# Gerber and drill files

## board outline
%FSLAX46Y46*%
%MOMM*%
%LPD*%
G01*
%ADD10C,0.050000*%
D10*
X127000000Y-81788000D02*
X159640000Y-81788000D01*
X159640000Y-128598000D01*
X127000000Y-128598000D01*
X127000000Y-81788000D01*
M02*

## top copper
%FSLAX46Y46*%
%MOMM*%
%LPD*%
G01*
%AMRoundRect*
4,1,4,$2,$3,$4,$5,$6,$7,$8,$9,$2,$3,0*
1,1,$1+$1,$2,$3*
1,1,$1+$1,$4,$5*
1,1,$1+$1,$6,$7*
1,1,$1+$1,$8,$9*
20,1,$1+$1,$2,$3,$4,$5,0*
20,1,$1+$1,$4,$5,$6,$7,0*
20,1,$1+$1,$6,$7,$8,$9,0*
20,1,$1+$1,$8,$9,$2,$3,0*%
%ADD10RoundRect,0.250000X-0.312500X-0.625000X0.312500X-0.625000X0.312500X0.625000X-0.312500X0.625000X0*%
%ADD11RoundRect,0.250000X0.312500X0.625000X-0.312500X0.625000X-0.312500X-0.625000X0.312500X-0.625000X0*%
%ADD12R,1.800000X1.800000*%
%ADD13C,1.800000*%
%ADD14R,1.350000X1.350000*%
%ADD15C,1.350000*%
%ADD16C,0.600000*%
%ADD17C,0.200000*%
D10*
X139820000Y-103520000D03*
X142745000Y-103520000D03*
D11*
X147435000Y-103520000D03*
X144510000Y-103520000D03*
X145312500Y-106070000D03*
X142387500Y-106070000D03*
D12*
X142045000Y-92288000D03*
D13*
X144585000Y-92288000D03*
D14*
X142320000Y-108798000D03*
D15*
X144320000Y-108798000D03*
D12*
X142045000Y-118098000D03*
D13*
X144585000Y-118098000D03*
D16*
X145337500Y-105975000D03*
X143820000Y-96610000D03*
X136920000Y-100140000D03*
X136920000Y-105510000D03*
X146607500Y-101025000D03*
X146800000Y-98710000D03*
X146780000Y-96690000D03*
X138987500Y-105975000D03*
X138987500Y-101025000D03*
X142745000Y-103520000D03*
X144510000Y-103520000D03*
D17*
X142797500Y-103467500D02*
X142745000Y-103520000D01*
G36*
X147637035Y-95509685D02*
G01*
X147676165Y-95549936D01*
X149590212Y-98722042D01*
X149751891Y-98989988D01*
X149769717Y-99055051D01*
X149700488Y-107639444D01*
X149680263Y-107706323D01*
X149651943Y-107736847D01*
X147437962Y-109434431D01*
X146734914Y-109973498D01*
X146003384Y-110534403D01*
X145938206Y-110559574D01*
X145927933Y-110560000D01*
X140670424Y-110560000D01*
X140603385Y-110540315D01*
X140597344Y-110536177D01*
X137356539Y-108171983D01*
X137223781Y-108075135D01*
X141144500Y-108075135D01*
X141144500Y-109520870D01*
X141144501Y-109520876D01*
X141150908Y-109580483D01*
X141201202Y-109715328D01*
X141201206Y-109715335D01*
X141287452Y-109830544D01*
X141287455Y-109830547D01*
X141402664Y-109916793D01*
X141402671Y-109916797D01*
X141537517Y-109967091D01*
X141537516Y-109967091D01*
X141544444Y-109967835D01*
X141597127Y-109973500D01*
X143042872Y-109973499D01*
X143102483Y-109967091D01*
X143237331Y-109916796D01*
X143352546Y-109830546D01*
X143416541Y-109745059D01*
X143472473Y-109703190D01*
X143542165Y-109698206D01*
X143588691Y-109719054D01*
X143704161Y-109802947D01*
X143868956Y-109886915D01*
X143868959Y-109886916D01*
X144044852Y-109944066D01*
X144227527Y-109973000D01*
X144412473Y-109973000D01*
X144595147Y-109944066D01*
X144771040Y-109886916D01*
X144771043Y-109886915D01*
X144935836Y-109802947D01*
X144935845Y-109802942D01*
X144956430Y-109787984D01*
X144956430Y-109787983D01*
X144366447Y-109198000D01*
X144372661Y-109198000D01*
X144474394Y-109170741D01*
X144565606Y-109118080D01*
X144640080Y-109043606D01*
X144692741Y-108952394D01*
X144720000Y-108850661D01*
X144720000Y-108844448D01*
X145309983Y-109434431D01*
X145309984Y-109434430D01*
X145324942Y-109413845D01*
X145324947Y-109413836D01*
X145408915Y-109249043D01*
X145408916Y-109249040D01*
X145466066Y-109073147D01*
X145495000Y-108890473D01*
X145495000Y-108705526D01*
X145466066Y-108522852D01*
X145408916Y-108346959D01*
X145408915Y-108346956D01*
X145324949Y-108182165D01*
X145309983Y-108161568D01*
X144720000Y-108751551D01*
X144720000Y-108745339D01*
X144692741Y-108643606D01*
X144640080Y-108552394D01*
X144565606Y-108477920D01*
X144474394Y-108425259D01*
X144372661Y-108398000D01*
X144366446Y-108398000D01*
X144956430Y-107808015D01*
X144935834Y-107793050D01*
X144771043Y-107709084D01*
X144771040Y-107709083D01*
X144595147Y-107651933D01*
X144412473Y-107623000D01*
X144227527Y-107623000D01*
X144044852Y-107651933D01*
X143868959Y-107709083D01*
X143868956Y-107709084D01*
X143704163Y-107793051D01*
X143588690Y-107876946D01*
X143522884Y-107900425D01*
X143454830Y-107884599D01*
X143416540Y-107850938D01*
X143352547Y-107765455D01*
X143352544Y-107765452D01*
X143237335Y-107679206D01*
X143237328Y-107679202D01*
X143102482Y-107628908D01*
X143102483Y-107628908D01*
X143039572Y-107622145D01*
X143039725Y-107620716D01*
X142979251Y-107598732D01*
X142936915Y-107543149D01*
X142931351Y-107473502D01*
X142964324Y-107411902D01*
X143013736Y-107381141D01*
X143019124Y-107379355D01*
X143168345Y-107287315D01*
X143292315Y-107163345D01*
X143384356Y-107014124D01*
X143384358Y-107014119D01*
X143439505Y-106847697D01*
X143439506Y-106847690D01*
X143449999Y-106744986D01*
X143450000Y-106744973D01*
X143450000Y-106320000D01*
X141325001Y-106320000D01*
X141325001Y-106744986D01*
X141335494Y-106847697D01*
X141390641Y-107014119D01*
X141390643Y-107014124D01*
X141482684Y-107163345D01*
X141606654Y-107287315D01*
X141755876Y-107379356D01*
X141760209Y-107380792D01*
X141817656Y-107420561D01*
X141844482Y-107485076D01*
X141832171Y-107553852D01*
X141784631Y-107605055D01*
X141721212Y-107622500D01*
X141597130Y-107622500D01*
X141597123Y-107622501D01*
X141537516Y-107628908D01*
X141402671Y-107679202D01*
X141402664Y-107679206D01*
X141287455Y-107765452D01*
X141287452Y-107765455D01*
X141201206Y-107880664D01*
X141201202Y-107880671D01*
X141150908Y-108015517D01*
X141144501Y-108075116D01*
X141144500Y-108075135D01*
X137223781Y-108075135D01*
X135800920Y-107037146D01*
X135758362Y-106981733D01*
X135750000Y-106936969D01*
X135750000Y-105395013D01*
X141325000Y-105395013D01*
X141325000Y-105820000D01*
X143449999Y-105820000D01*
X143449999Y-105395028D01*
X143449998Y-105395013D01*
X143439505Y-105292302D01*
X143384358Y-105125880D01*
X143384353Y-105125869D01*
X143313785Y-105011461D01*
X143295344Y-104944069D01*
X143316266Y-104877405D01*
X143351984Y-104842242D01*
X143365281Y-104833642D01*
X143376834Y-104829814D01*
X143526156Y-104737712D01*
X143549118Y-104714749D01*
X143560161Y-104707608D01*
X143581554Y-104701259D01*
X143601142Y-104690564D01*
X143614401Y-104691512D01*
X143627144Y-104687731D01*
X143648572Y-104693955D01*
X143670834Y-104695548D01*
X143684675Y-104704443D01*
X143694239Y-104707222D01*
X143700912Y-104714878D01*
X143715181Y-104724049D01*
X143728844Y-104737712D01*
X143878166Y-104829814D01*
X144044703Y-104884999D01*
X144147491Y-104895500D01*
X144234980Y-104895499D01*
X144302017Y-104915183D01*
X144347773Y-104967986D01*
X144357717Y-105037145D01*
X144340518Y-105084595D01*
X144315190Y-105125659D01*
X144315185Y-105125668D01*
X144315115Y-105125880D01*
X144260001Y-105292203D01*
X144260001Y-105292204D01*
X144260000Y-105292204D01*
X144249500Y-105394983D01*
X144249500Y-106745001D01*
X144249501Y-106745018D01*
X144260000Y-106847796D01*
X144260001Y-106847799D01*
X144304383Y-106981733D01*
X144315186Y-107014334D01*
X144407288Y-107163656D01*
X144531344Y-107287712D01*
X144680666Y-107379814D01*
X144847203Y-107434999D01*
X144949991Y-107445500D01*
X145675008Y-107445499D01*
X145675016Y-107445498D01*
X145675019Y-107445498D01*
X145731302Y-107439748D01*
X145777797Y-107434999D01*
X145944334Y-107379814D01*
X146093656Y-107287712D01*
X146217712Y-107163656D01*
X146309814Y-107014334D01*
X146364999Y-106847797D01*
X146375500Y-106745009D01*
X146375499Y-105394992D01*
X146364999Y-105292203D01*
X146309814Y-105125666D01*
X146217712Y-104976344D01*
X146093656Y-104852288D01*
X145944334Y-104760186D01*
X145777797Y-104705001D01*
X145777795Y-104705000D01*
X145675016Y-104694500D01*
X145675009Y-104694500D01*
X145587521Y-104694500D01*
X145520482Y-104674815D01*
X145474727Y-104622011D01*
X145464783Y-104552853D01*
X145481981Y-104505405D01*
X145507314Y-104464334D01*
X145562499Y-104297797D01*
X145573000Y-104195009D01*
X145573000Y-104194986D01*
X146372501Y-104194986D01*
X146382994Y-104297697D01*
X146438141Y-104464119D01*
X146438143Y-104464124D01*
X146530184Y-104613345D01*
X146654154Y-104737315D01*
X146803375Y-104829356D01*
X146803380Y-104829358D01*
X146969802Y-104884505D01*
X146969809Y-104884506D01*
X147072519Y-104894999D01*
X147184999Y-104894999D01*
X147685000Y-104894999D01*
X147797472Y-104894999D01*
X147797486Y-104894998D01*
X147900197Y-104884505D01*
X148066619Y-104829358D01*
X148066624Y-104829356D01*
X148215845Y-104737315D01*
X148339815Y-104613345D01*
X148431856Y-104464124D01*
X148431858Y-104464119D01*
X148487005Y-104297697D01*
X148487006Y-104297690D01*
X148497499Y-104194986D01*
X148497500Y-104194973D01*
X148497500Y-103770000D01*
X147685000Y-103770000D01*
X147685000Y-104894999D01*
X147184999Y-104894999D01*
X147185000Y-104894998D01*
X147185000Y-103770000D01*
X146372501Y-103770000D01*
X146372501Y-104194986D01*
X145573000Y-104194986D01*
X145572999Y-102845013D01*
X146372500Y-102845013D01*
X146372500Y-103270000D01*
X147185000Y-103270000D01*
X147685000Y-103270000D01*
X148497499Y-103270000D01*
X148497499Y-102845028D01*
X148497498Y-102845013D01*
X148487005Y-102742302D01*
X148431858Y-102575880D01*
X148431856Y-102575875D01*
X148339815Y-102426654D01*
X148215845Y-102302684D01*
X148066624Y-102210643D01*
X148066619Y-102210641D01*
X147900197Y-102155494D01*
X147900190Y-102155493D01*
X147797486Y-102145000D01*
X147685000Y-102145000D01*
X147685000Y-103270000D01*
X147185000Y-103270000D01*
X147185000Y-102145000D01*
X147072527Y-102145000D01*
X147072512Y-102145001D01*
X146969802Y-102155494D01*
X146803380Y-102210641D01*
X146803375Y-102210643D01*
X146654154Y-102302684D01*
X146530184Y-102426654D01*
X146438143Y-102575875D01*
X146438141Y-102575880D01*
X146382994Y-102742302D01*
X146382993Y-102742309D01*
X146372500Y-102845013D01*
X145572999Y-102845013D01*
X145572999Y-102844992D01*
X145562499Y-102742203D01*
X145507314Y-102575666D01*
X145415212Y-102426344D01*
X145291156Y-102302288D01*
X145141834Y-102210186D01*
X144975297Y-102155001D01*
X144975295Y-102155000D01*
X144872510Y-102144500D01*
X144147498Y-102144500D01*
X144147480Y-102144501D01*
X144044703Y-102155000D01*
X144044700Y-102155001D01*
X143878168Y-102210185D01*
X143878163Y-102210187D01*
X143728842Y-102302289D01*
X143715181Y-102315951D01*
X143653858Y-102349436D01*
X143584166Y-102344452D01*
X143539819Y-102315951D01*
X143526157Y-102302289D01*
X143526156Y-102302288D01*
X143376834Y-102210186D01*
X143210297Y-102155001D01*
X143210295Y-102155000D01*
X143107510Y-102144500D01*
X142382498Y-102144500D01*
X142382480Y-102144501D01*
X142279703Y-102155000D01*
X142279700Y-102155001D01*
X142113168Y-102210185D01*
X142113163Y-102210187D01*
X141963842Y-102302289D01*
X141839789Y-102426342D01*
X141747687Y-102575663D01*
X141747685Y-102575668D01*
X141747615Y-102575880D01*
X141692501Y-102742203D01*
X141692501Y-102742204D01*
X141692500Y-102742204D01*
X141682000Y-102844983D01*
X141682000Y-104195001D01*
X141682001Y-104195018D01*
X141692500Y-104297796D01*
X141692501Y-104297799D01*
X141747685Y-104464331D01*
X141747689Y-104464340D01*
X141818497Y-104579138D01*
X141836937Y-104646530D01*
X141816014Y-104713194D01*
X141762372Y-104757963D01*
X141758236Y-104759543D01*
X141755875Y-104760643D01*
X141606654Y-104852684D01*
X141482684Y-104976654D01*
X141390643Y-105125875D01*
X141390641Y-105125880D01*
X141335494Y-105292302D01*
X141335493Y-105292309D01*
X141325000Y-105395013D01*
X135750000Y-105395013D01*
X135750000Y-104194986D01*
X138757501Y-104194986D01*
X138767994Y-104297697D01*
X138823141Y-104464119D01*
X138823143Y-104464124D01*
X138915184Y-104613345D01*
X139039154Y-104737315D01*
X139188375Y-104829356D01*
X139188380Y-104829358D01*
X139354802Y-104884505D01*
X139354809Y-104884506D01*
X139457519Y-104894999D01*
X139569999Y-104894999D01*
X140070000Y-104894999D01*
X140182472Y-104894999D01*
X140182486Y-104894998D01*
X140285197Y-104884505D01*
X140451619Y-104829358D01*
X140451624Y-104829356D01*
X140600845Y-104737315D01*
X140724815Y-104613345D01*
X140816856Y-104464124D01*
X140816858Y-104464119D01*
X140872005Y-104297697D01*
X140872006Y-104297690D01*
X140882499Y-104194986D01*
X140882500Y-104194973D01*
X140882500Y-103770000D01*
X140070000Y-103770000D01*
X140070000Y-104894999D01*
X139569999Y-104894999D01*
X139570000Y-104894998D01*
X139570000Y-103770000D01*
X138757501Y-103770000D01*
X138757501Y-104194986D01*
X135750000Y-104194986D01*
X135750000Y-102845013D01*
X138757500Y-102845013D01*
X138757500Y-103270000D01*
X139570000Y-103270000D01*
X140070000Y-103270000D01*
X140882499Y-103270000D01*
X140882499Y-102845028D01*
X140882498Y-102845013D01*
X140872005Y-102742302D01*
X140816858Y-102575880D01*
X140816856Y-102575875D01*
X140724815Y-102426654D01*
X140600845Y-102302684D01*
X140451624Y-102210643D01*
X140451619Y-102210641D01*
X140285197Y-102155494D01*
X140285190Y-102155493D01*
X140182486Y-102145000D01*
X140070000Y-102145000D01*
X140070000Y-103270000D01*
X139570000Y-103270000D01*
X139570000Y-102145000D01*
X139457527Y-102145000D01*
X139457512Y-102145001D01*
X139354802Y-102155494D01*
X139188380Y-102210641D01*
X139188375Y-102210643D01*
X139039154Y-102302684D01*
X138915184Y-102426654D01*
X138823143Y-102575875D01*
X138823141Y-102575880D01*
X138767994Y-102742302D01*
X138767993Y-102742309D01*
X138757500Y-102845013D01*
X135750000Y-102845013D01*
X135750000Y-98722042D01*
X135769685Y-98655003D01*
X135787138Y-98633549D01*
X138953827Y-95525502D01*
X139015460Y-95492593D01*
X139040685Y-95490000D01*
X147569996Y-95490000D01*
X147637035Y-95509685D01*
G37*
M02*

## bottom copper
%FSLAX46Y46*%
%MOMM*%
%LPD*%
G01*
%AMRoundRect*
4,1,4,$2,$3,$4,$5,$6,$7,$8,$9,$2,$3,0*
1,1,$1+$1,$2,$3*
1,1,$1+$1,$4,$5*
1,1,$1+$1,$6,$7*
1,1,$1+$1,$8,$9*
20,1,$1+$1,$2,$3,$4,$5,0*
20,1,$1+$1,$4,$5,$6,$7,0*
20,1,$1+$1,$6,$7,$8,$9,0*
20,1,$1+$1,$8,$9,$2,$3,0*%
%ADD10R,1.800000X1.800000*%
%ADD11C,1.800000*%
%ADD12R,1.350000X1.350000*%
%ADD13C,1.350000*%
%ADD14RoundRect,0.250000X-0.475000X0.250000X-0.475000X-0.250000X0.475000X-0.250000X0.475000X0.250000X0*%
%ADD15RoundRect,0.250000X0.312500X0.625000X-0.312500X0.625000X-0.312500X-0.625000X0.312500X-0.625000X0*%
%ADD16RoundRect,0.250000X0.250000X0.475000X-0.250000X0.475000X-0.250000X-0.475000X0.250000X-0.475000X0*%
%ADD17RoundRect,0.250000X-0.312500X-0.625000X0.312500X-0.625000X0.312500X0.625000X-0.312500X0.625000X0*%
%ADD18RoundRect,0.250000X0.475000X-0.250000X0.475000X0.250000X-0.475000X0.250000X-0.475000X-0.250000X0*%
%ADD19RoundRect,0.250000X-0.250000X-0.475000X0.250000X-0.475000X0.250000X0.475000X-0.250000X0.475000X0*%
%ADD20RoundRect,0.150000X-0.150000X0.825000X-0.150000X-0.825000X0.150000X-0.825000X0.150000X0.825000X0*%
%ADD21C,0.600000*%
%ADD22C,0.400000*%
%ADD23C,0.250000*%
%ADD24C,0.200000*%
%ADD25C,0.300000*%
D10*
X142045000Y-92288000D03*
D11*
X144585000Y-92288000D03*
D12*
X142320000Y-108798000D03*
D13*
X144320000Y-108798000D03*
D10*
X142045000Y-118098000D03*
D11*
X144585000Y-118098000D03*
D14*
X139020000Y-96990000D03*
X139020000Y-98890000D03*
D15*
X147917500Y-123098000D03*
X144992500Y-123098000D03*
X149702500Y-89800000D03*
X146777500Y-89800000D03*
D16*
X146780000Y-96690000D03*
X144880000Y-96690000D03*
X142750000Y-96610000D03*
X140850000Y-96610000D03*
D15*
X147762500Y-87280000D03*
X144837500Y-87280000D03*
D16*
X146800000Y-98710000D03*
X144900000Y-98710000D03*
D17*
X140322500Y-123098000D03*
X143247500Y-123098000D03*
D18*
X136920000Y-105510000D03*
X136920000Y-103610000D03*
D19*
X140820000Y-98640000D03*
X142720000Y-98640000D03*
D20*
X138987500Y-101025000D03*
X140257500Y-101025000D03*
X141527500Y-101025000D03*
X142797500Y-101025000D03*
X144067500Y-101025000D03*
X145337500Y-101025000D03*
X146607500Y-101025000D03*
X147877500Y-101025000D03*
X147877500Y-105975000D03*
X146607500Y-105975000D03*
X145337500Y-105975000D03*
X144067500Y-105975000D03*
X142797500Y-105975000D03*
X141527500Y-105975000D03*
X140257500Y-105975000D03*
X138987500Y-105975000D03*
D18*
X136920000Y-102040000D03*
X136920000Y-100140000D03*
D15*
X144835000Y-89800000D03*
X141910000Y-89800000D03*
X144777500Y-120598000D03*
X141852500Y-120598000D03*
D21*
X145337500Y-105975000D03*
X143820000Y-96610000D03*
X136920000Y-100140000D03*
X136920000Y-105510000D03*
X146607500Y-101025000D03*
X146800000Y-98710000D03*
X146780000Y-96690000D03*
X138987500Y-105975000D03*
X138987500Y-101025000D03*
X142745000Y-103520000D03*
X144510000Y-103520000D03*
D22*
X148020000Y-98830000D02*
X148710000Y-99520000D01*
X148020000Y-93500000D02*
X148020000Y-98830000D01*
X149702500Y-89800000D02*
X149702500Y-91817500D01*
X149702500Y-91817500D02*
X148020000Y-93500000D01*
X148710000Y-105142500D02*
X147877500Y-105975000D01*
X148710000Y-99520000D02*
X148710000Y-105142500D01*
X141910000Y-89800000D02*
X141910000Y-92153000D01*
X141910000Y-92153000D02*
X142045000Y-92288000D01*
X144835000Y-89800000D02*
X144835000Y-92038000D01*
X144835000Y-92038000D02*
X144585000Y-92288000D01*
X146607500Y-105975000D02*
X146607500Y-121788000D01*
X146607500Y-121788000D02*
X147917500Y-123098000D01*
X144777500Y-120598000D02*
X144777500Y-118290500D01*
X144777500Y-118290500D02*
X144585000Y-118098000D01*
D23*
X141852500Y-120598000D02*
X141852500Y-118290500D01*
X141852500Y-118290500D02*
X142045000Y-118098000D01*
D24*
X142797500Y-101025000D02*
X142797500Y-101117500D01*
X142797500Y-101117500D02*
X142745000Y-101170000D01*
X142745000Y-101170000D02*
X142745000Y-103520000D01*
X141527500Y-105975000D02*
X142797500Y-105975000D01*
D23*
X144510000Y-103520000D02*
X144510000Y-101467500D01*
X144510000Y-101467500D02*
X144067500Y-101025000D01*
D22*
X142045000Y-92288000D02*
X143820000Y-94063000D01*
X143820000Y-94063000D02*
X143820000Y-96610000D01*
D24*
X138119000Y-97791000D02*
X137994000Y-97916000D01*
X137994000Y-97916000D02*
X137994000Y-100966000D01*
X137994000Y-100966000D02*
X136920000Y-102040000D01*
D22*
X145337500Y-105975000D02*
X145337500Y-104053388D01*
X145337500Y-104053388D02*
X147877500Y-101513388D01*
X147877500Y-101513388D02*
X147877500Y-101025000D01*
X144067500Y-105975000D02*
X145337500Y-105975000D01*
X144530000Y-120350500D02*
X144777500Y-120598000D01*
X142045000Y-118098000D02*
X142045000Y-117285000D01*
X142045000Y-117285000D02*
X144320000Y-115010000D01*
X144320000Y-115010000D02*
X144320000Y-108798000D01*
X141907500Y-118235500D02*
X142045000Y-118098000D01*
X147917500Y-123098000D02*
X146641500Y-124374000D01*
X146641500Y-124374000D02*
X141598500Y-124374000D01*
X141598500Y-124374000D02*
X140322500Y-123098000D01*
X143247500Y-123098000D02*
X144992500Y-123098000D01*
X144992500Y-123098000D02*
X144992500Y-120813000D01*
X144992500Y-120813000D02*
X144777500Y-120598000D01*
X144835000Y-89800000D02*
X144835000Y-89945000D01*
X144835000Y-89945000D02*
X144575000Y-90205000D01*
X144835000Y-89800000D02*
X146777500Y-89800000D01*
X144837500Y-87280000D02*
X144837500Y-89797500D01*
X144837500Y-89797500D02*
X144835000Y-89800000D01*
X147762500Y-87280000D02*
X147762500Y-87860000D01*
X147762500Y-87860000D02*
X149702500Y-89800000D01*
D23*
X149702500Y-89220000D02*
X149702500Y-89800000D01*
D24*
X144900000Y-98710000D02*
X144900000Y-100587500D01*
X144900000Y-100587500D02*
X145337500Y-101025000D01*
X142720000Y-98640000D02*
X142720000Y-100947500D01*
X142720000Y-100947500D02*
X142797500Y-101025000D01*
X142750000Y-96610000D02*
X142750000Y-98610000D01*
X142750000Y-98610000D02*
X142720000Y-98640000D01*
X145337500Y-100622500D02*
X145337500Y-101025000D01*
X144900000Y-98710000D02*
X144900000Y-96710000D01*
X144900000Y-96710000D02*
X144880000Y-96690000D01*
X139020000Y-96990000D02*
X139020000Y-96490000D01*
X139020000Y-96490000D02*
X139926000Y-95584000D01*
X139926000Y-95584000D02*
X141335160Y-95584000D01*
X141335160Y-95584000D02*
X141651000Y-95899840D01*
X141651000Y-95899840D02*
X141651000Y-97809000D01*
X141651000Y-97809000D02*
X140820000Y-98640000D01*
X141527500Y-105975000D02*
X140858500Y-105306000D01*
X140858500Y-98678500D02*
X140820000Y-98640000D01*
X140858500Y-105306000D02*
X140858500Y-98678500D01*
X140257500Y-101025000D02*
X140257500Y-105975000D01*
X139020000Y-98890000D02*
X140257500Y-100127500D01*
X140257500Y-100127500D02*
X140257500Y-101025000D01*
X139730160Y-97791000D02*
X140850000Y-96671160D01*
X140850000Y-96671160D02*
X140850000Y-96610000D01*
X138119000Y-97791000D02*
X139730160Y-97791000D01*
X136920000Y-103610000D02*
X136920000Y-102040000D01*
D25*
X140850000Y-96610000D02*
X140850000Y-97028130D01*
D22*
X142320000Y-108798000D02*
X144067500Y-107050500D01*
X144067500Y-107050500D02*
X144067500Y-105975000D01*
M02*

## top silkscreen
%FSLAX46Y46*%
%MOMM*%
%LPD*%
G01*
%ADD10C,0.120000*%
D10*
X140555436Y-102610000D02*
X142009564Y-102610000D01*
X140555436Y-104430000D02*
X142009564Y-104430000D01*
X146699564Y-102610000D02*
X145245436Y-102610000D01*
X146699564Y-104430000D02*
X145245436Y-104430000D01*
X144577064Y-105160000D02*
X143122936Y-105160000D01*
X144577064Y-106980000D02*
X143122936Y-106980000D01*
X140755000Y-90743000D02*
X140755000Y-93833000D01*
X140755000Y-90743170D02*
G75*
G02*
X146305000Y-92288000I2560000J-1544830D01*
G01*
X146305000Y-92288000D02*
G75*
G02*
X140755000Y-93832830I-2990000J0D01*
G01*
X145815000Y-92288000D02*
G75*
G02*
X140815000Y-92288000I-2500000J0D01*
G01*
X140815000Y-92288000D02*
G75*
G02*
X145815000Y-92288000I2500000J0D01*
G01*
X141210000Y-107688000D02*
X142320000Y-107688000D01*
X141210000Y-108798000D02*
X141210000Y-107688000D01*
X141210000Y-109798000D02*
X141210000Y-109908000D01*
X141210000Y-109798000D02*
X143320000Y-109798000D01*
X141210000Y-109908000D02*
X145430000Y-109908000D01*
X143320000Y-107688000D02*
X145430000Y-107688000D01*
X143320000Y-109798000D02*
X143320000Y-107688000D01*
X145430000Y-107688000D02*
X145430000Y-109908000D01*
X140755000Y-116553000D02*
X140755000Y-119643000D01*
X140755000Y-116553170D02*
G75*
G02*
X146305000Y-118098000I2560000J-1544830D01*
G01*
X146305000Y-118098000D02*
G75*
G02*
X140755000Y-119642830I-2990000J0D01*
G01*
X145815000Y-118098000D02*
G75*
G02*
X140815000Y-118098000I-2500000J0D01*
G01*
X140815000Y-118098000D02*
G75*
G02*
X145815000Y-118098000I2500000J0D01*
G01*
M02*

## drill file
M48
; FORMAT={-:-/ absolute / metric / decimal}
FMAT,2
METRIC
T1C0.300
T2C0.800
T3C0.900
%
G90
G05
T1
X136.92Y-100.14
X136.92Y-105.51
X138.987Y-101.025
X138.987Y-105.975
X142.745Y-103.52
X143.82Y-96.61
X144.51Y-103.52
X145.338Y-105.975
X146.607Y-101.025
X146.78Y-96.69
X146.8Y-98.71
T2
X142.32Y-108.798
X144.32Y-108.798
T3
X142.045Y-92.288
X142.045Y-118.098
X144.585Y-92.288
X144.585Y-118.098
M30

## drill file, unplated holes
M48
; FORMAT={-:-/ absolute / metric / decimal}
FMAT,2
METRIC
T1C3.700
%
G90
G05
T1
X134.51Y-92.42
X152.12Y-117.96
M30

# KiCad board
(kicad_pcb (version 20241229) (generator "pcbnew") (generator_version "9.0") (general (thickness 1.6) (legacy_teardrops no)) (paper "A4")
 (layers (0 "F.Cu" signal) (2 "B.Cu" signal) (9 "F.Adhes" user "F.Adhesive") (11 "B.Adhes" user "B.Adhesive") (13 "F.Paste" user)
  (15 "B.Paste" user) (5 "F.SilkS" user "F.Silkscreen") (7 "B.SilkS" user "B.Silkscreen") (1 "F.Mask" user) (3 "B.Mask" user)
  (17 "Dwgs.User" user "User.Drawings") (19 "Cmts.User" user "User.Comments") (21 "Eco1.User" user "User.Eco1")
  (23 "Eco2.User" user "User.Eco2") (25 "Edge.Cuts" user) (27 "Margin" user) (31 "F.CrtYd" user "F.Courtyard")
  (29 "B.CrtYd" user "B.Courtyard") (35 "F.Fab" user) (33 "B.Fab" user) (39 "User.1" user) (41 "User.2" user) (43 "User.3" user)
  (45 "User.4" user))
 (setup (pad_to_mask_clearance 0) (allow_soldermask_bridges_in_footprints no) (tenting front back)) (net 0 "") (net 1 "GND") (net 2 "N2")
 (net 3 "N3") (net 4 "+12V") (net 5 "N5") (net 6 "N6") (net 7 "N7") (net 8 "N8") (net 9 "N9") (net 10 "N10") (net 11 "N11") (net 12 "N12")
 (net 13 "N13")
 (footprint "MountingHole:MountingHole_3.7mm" (layer "F.Cu") (at 152.12 117.96)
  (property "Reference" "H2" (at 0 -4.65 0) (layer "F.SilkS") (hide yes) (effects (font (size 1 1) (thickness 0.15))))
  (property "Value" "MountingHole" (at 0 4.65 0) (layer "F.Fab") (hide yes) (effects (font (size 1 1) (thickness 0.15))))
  (pad "" np_thru_hole circle (at 0 0) (size 3.7 3.7) (drill 3.7) (layers "*.Cu" "*.Mask")))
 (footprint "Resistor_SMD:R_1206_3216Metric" (layer "F.Cu") (at 141.2825 103.52)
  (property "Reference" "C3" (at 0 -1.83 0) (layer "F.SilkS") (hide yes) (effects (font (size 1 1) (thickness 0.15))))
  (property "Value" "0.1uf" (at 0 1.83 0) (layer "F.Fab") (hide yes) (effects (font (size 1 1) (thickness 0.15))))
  (fp_line (start -0.727064 -0.91) (end 0.727064 -0.91) (stroke (width 0.12) (type solid)) (layer "F.SilkS"))
  (fp_line (start -0.727064 0.91) (end 0.727064 0.91) (stroke (width 0.12) (type solid)) (layer "F.SilkS"))
  (pad "1" smd roundrect (at -1.4625 0) (size 1.125 1.75) (layers "F.Cu" "F.Mask" "F.Paste") (roundrect_rratio 0.222222) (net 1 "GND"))
  (pad "2" smd roundrect (at 1.4625 0) (size 1.125 1.75) (layers "F.Cu" "F.Mask" "F.Paste") (roundrect_rratio 0.222222) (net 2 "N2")))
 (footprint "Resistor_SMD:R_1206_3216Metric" (layer "F.Cu") (at 145.9725 103.52 180)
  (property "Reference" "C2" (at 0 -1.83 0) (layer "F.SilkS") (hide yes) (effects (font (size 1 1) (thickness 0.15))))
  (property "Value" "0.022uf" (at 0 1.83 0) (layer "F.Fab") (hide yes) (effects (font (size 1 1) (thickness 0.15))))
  (fp_line (start -0.727064 0.91) (end 0.727064 0.91) (stroke (width 0.12) (type solid)) (layer "F.SilkS"))
  (fp_line (start -0.727064 -0.91) (end 0.727064 -0.91) (stroke (width 0.12) (type solid)) (layer "F.SilkS"))
  (pad "1" smd roundrect (at -1.4625 0 180) (size 1.125 1.75) (layers "F.Cu" "F.Mask" "F.Paste") (roundrect_rratio 0.222222) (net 1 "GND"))
  (pad "2" smd roundrect (at 1.4625 0 180) (size 1.125 1.75) (layers "F.Cu" "F.Mask" "F.Paste") (roundrect_rratio 0.222222) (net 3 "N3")))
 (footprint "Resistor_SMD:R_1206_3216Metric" (layer "F.Cu") (at 143.85 106.07 180)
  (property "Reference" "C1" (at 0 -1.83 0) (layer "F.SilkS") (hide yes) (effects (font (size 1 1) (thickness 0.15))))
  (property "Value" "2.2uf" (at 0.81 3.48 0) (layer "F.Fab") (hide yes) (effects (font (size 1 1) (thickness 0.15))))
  (fp_line (start -0.727064 0.91) (end 0.727064 0.91) (stroke (width 0.12) (type solid)) (layer "F.SilkS"))
  (fp_line (start -0.727064 -0.91) (end 0.727064 -0.91) (stroke (width 0.12) (type solid)) (layer "F.SilkS"))
  (pad "1" smd roundrect (at -1.4625 0 180) (size 1.125 1.75) (layers "F.Cu" "F.Mask" "F.Paste") (roundrect_rratio 0.222222) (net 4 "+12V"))
  (pad "2" smd roundrect (at 1.4625 0 180) (size 1.125 1.75) (layers "F.Cu" "F.Mask" "F.Paste") (roundrect_rratio 0.222222) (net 1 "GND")))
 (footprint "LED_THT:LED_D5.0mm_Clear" (layer "F.Cu") (at 142.045 92.288)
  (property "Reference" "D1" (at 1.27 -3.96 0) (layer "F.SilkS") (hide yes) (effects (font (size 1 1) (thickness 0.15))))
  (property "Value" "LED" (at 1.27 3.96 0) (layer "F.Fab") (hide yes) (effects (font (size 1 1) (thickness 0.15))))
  (fp_line (start -1.29 -1.545) (end -1.29 1.545) (stroke (width 0.12) (type solid)) (layer "F.SilkS"))
  (fp_arc (start -1.29 -1.54483) (mid 2.071779 -2.880495) (end 4.26 0) (stroke (width 0.12) (type solid)) (layer "F.SilkS"))
  (fp_arc (start 4.26 0) (mid 2.071779 2.880495) (end -1.29 1.54483) (stroke (width 0.12) (type solid)) (layer "F.SilkS"))
  (fp_circle (center 1.27 0) (end 3.77 0) (stroke (width 0.12) (type solid)) (fill no) (layer "F.SilkS"))
  (pad "1" thru_hole rect (at 0 0) (size 1.8 1.8) (drill 0.9) (layers "*.Cu" "*.Mask") (remove_unused_layers no) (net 1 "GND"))
  (pad "2" thru_hole circle (at 2.54 0) (size 1.8 1.8) (drill 0.9) (layers "*.Cu" "*.Mask") (remove_unused_layers no) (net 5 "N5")))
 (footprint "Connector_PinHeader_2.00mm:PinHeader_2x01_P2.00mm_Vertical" (layer "F.Cu") (at 142.32 108.798)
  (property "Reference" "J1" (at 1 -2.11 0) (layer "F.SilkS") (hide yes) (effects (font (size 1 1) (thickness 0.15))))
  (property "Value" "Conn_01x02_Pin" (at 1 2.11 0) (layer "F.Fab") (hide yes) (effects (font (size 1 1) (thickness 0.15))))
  (fp_line (start -1.11 -1.11) (end 0 -1.11) (stroke (width 0.12) (type solid)) (layer "F.SilkS"))
  (fp_line (start -1.11 0) (end -1.11 -1.11) (stroke (width 0.12) (type solid)) (layer "F.SilkS"))
  (fp_line (start -1.11 1) (end -1.11 1.11) (stroke (width 0.12) (type solid)) (layer "F.SilkS"))
  (fp_line (start -1.11 1) (end 1 1) (stroke (width 0.12) (type solid)) (layer "F.SilkS"))
  (fp_line (start -1.11 1.11) (end 3.11 1.11) (stroke (width 0.12) (type solid)) (layer "F.SilkS"))
  (fp_line (start 1 -1.11) (end 3.11 -1.11) (stroke (width 0.12) (type solid)) (layer "F.SilkS"))
  (fp_line (start 1 1) (end 1 -1.11) (stroke (width 0.12) (type solid)) (layer "F.SilkS"))
  (fp_line (start 3.11 -1.11) (end 3.11 1.11) (stroke (width 0.12) (type solid)) (layer "F.SilkS"))
  (pad "1" thru_hole rect (at 0 0) (size 1.35 1.35) (drill 0.8) (layers "*.Cu" "*.Mask") (remove_unused_layers no) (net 4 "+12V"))
  (pad "2" thru_hole circle (at 2 0) (size 1.35 1.35) (drill 0.8) (layers "*.Cu" "*.Mask") (remove_unused_layers no) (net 1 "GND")))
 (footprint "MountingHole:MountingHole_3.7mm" (layer "F.Cu") (at 134.51 92.42)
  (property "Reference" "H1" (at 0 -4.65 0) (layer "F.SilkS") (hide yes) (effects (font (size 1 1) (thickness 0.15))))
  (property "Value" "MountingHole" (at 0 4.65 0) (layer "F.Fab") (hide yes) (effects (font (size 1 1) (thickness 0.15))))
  (pad "" np_thru_hole circle (at 0 0) (size 3.7 3.7) (drill 3.7) (layers "*.Cu" "*.Mask")))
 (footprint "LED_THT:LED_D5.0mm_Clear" (layer "F.Cu") (at 142.045 118.098)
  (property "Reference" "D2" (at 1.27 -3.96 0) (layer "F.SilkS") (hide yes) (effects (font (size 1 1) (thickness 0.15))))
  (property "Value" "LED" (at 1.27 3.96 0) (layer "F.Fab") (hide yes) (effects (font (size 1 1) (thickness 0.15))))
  (fp_line (start -1.29 -1.545) (end -1.29 1.545) (stroke (width 0.12) (type solid)) (layer "F.SilkS"))
  (fp_arc (start -1.29 -1.54483) (mid 2.071779 -2.880495) (end 4.26 0) (stroke (width 0.12) (type solid)) (layer "F.SilkS"))
  (fp_arc (start 4.26 0) (mid 2.071779 2.880495) (end -1.29 1.54483) (stroke (width 0.12) (type solid)) (layer "F.SilkS"))
  (fp_circle (center 1.27 0) (end 3.77 0) (stroke (width 0.12) (type solid)) (fill no) (layer "F.SilkS"))
  (pad "1" thru_hole rect (at 0 0) (size 1.8 1.8) (drill 0.9) (layers "*.Cu" "*.Mask") (remove_unused_layers no) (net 1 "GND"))
  (pad "2" thru_hole circle (at 2.54 0) (size 1.8 1.8) (drill 0.9) (layers "*.Cu" "*.Mask") (remove_unused_layers no) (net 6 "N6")))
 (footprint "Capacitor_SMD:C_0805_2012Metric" (layer "B.Cu") (at 139.02 97.94 -90)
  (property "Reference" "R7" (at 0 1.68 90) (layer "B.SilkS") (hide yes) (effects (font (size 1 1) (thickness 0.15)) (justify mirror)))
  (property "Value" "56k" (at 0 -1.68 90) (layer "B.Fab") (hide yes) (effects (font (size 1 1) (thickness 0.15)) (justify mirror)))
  (pad "1" smd roundrect (at -0.95 0 270) (size 1 1.45) (layers "B.Cu" "B.Mask" "B.Paste") (roundrect_rratio 0.25) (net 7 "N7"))
  (pad "2" smd roundrect (at 0.95 0 270) (size 1 1.45) (layers "B.Cu" "B.Mask" "B.Paste") (roundrect_rratio 0.25) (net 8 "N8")))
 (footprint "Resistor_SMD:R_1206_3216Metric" (layer "B.Cu") (at 146.455 123.098 180)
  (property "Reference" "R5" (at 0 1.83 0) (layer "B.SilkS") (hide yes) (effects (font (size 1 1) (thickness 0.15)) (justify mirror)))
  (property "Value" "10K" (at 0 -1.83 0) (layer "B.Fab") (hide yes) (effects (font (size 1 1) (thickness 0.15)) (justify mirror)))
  (pad "1" smd roundrect (at -1.4625 0 180) (size 1.125 1.75) (layers "B.Cu" "B.Mask" "B.Paste") (roundrect_rratio 0.222222) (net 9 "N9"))
  (pad "2" smd roundrect (at 1.4625 0 180) (size 1.125 1.75) (layers "B.Cu" "B.Mask" "B.Paste") (roundrect_rratio 0.222222) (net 6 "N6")))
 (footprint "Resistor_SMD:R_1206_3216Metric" (layer "B.Cu") (at 148.24 89.8 180)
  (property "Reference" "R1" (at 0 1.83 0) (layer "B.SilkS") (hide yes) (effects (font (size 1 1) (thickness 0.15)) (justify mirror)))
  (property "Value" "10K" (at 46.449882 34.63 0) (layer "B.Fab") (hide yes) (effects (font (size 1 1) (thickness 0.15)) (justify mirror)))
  (pad "1" smd roundrect (at -1.4625 0 180) (size 1.125 1.75) (layers "B.Cu" "B.Mask" "B.Paste") (roundrect_rratio 0.222222) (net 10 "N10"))
  (pad "2" smd roundrect (at 1.4625 0 180) (size 1.125 1.75) (layers "B.Cu" "B.Mask" "B.Paste") (roundrect_rratio 0.222222) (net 5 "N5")))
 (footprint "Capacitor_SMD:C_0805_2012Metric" (layer "B.Cu") (at 145.83 96.69 180)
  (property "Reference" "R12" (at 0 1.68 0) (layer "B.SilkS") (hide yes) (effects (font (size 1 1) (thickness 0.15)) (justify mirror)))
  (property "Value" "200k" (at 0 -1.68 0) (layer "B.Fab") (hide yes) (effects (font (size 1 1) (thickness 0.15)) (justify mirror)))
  (pad "1" smd roundrect (at -0.95 0 180) (size 1 1.45) (layers "B.Cu" "B.Mask" "B.Paste") (roundrect_rratio 0.25) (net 1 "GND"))
  (pad "2" smd roundrect (at 0.95 0 180) (size 1 1.45) (layers "B.Cu" "B.Mask" "B.Paste") (roundrect_rratio 0.25) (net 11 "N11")))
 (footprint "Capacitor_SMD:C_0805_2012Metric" (layer "B.Cu") (at 141.8 96.61 180)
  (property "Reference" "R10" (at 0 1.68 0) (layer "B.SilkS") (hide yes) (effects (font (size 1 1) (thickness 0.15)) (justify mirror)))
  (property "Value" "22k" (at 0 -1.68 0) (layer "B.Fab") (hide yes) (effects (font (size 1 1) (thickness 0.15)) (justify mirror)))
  (pad "1" smd roundrect (at -0.95 0 180) (size 1 1.45) (layers "B.Cu" "B.Mask" "B.Paste") (roundrect_rratio 0.25) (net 2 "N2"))
  (pad "2" smd roundrect (at 0.95 0 180) (size 1 1.45) (layers "B.Cu" "B.Mask" "B.Paste") (roundrect_rratio 0.25) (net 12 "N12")))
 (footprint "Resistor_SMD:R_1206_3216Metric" (layer "B.Cu") (at 146.3 87.28 180)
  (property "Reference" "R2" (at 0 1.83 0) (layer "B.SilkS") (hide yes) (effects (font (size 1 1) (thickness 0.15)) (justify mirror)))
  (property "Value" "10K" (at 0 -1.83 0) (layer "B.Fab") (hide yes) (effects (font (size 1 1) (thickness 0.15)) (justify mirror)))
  (pad "1" smd roundrect (at -1.4625 0 180) (size 1.125 1.75) (layers "B.Cu" "B.Mask" "B.Paste") (roundrect_rratio 0.222222) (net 10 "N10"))
  (pad "2" smd roundrect (at 1.4625 0 180) (size 1.125 1.75) (layers "B.Cu" "B.Mask" "B.Paste") (roundrect_rratio 0.222222) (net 5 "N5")))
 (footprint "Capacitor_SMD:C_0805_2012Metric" (layer "B.Cu") (at 145.85 98.71 180)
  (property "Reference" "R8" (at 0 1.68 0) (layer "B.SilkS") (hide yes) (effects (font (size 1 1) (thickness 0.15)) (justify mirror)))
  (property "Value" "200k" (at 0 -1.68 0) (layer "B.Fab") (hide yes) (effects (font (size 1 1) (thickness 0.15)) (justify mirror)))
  (pad "1" smd roundrect (at -0.95 0 180) (size 1 1.45) (layers "B.Cu" "B.Mask" "B.Paste") (roundrect_rratio 0.25) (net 1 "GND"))
  (pad "2" smd roundrect (at 0.95 0 180) (size 1 1.45) (layers "B.Cu" "B.Mask" "B.Paste") (roundrect_rratio 0.25) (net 11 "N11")))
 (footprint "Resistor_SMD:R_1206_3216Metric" (layer "B.Cu") (at 141.785 123.098)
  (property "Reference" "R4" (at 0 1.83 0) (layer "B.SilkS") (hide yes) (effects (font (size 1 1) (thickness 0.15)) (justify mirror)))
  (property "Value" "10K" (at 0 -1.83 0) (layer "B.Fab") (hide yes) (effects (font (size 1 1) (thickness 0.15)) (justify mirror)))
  (pad "1" smd roundrect (at -1.4625 0) (size 1.125 1.75) (layers "B.Cu" "B.Mask" "B.Paste") (roundrect_rratio 0.222222) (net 9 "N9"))
  (pad "2" smd roundrect (at 1.4625 0) (size 1.125 1.75) (layers "B.Cu" "B.Mask" "B.Paste") (roundrect_rratio 0.222222) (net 6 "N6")))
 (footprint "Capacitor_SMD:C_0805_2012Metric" (layer "B.Cu") (at 136.92 104.56 90)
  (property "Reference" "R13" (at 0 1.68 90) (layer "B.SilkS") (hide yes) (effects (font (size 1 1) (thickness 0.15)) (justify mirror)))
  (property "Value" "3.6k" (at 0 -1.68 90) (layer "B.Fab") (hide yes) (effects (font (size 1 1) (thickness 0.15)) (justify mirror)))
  (pad "1" smd roundrect (at -0.95 0 90) (size 1 1.45) (layers "B.Cu" "B.Mask" "B.Paste") (roundrect_rratio 0.25) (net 1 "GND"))
  (pad "2" smd roundrect (at 0.95 0 90) (size 1 1.45) (layers "B.Cu" "B.Mask" "B.Paste") (roundrect_rratio 0.25) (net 12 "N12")))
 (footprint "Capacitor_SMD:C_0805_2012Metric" (layer "B.Cu") (at 141.77 98.64)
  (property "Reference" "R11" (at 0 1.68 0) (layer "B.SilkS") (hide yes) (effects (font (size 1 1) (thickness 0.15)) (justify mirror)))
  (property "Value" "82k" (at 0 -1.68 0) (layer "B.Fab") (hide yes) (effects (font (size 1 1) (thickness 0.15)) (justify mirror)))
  (pad "1" smd roundrect (at -0.95 0) (size 1 1.45) (layers "B.Cu" "B.Mask" "B.Paste") (roundrect_rratio 0.25) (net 7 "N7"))
  (pad "2" smd roundrect (at 0.95 0) (size 1 1.45) (layers "B.Cu" "B.Mask" "B.Paste") (roundrect_rratio 0.25) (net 2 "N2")))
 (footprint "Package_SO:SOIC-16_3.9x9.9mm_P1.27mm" (layer "B.Cu") (at 143.4325 103.5 -90)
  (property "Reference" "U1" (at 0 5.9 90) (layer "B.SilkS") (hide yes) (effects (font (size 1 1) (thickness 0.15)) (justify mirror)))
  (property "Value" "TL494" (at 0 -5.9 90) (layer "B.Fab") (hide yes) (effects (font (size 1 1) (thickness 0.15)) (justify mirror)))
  (pad "1" smd roundrect (at -2.475 4.445 270) (size 1.95 0.6) (layers "B.Cu" "B.Mask" "B.Paste") (roundrect_rratio 0.25) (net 1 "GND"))
  (pad "2" smd roundrect (at -2.475 3.175 270) (size 1.95 0.6) (layers "B.Cu" "B.Mask" "B.Paste") (roundrect_rratio 0.25) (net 8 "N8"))
  (pad "3" smd roundrect (at -2.475 1.905 270) (size 1.95 0.6) (layers "B.Cu" "B.Mask" "B.Paste") (roundrect_rratio 0.25) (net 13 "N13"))
  (pad "4" smd roundrect (at -2.475 0.635 270) (size 1.95 0.6) (layers "B.Cu" "B.Mask" "B.Paste") (roundrect_rratio 0.25) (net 2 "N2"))
  (pad "5" smd roundrect (at -2.475 -0.635 270) (size 1.95 0.6) (layers "B.Cu" "B.Mask" "B.Paste") (roundrect_rratio 0.25) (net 3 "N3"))
  (pad "6" smd roundrect (at -2.475 -1.905 270) (size 1.95 0.6) (layers "B.Cu" "B.Mask" "B.Paste") (roundrect_rratio 0.25) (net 11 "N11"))
  (pad "7" smd roundrect (at -2.475 -3.175 270) (size 1.95 0.6) (layers "B.Cu" "B.Mask" "B.Paste") (roundrect_rratio 0.25) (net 1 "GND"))
  (pad "8" smd roundrect (at -2.475 -4.445 270) (size 1.95 0.6) (layers "B.Cu" "B.Mask" "B.Paste") (roundrect_rratio 0.25) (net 4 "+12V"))
  (pad "9" smd roundrect (at 2.475 -4.445 270) (size 1.95 0.6) (layers "B.Cu" "B.Mask" "B.Paste") (roundrect_rratio 0.25) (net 10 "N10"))
  (pad "10" smd roundrect (at 2.475 -3.175 270) (size 1.95 0.6) (layers "B.Cu" "B.Mask" "B.Paste") (roundrect_rratio 0.25) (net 9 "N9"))
  (pad "11" smd roundrect (at 2.475 -1.905 270) (size 1.95 0.6) (layers "B.Cu" "B.Mask" "B.Paste") (roundrect_rratio 0.25) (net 4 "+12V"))
  (pad "12" smd roundrect (at 2.475 -0.635 270) (size 1.95 0.6) (layers "B.Cu" "B.Mask" "B.Paste") (roundrect_rratio 0.25) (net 4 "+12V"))
  (pad "13" smd roundrect (at 2.475 0.635 270) (size 1.95 0.6) (layers "B.Cu" "B.Mask" "B.Paste") (roundrect_rratio 0.25) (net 7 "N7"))
  (pad "14" smd roundrect (at 2.475 1.905 270) (size 1.95 0.6) (layers "B.Cu" "B.Mask" "B.Paste") (roundrect_rratio 0.25) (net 7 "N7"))
  (pad "15" smd roundrect (at 2.475 3.175 270) (size 1.95 0.6) (layers "B.Cu" "B.Mask" "B.Paste") (roundrect_rratio 0.25) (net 8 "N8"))
  (pad "16" smd roundrect (at 2.475 4.445 270) (size 1.95 0.6) (layers "B.Cu" "B.Mask" "B.Paste") (roundrect_rratio 0.25) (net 1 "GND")))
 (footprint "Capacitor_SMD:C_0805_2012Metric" (layer "B.Cu") (at 136.92 101.09 90)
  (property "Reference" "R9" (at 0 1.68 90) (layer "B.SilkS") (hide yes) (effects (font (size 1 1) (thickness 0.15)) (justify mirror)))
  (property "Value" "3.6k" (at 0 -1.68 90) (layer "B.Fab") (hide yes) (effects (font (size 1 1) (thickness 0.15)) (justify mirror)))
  (pad "1" smd roundrect (at -0.95 0 90) (size 1 1.45) (layers "B.Cu" "B.Mask" "B.Paste") (roundrect_rratio 0.25) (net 12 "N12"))
  (pad "2" smd roundrect (at 0.95 0 90) (size 1 1.45) (layers "B.Cu" "B.Mask" "B.Paste") (roundrect_rratio 0.25) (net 1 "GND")))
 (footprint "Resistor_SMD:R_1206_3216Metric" (layer "B.Cu") (at 143.3725 89.8 180)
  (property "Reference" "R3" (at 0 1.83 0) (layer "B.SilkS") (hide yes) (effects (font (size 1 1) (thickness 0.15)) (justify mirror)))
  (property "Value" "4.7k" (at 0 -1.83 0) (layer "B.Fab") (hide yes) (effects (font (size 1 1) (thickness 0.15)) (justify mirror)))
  (pad "1" smd roundrect (at -1.4625 0 180) (size 1.125 1.75) (layers "B.Cu" "B.Mask" "B.Paste") (roundrect_rratio 0.222222) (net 5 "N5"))
  (pad "2" smd roundrect (at 1.4625 0 180) (size 1.125 1.75) (layers "B.Cu" "B.Mask" "B.Paste") (roundrect_rratio 0.222222) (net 1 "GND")))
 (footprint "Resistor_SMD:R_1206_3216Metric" (layer "B.Cu") (at 143.315 120.598 180)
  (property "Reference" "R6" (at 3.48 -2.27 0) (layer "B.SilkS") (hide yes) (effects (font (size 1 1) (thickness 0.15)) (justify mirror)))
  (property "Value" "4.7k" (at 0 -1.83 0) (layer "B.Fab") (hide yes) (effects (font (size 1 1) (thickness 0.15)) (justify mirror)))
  (pad "1" smd roundrect (at -1.4625 0 180) (size 1.125 1.75) (layers "B.Cu" "B.Mask" "B.Paste") (roundrect_rratio 0.222222) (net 6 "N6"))
  (pad "2" smd roundrect (at 1.4625 0 180) (size 1.125 1.75) (layers "B.Cu" "B.Mask" "B.Paste") (roundrect_rratio 0.222222) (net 1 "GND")))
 (gr_rect (start 127 81.788) (end 159.64 128.598) (stroke (width 0.05) (type default)) (fill no) (layer "Edge.Cuts"))
 (via (at 145.3375 105.975) (size 0.6) (drill 0.3) (layers "F.Cu" "B.Cu") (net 4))
 (segment (start 147.8775 101.513388) (end 147.8775 101.025) (width 0.4) (layer "B.Cu") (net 4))
 (segment (start 144.0675 107.0505) (end 144.0675 105.975) (width 0.4) (layer "B.Cu") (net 4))
 (segment (start 142.32 108.798) (end 144.0675 107.0505) (width 0.4) (layer "B.Cu") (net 4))
 (segment (start 145.3375 104.053388) (end 147.8775 101.513388) (width 0.4) (layer "B.Cu") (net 4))
 (segment (start 144.0675 105.975) (end 145.3375 105.975) (width 0.4) (layer "B.Cu") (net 4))
 (segment (start 145.3375 105.975) (end 145.3375 104.053388) (width 0.4) (layer "B.Cu") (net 4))
 (via (at 138.9875 105.975) (size 0.6) (drill 0.3) (layers "F.Cu" "B.Cu") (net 1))
 (via (at 146.78 96.69) (size 0.6) (drill 0.3) (layers "F.Cu" "B.Cu") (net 1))
 (via (at 146.6075 101.025) (size 0.6) (drill 0.3) (layers "F.Cu" "B.Cu") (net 1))
 (via (at 138.9875 101.025) (size 0.6) (drill 0.3) (layers "F.Cu" "B.Cu") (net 1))
 (via (at 146.8 98.71) (size 0.6) (drill 0.3) (layers "F.Cu" "B.Cu") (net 1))
 (via (at 136.92 100.14) (size 0.6) (drill 0.3) (layers "F.Cu" "B.Cu") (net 1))
 (via (at 143.82 96.61) (size 0.6) (drill 0.3) (layers "F.Cu" "B.Cu") (free yes) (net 1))
 (via (at 136.92 105.51) (size 0.6) (drill 0.3) (layers "F.Cu" "B.Cu") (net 1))
 (segment (start 142.045 92.288) (end 143.82 94.063) (width 0.4) (layer "B.Cu") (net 1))
 (segment (start 141.9075 118.2355) (end 142.045 118.098) (width 0.4) (layer "B.Cu") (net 1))
 (segment (start 142.045 117.285) (end 144.32 115.01) (width 0.4) (layer "B.Cu") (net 1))
 (segment (start 141.8525 118.2905) (end 142.045 118.098) (width 0.25) (layer "B.Cu") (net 1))
 (segment (start 141.91 92.153) (end 142.045 92.288) (width 0.4) (layer "B.Cu") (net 1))
 (segment (start 143.82 94.063) (end 143.82 96.61) (width 0.4) (layer "B.Cu") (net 1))
 (segment (start 142.045 118.098) (end 142.045 117.285) (width 0.4) (layer "B.Cu") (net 1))
 (segment (start 144.32 115.01) (end 144.32 108.798) (width 0.4) (layer "B.Cu") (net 1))
 (segment (start 141.8525 120.598) (end 141.8525 118.2905) (width 0.25) (layer "B.Cu") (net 1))
 (segment (start 141.91 89.8) (end 141.91 92.153) (width 0.4) (layer "B.Cu") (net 1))
 (via (at 144.51 103.52) (size 0.6) (drill 0.3) (layers "F.Cu" "B.Cu") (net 3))
 (segment (start 144.51 101.4675) (end 144.0675 101.025) (width 0.25) (layer "B.Cu") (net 3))
 (segment (start 144.51 103.52) (end 144.51 101.4675) (width 0.25) (layer "B.Cu") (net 3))
 (segment (start 140.8585 98.6785) (end 140.82 98.64) (width 0.2) (layer "B.Cu") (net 7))
 (segment (start 140.8585 105.306) (end 140.8585 98.6785) (width 0.2) (layer "B.Cu") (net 7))
 (segment (start 141.651 95.89984) (end 141.651 97.809) (width 0.2) (layer "B.Cu") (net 7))
 (segment (start 139.02 96.99) (end 139.02 96.49) (width 0.2) (layer "B.Cu") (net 7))
 (segment (start 139.02 96.49) (end 139.926 95.584) (width 0.2) (layer "B.Cu") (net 7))
 (segment (start 141.651 97.809) (end 140.82 98.64) (width 0.2) (layer "B.Cu") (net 7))
 (segment (start 141.5275 105.975) (end 140.8585 105.306) (width 0.2) (layer "B.Cu") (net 7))
 (segment (start 141.5275 105.975) (end 142.7975 105.975) (width 0.2) (layer "B.Cu") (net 7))
 (segment (start 139.926 95.584) (end 141.33516 95.584) (width 0.2) (layer "B.Cu") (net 7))
 (segment (start 141.33516 95.584) (end 141.651 95.89984) (width 0.2) (layer "B.Cu") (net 7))
 (segment (start 144.8375 87.28) (end 144.8375 89.7975) (width 0.4) (layer "B.Cu") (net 5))
 (segment (start 144.8375 89.7975) (end 144.835 89.8) (width 0.4) (layer "B.Cu") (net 5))
 (segment (start 144.835 89.8) (end 146.7775 89.8) (width 0.4) (layer "B.Cu") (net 5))
 (segment (start 144.835 92.038) (end 144.585 92.288) (width 0.4) (layer "B.Cu") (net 5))
 (segment (start 144.835 89.8) (end 144.835 92.038) (width 0.4) (layer "B.Cu") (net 5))
 (segment (start 144.835 89.945) (end 144.575 90.205) (width 0.4) (layer "B.Cu") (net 5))
 (segment (start 144.835 89.8) (end 144.835 89.945) (width 0.4) (layer "B.Cu") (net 5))
 (segment (start 144.9925 123.098) (end 144.9925 120.813) (width 0.4) (layer "B.Cu") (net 6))
 (segment (start 143.2475 123.098) (end 144.9925 123.098) (width 0.4) (layer "B.Cu") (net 6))
 (segment (start 144.7775 118.2905) (end 144.585 118.098) (width 0.4) (layer "B.Cu") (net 6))
 (segment (start 144.53 120.3505) (end 144.7775 120.598) (width 0.4) (layer "B.Cu") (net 6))
 (segment (start 144.9925 120.813) (end 144.7775 120.598) (width 0.4) (layer "B.Cu") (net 6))
 (segment (start 144.7775 120.598) (end 144.7775 118.2905) (width 0.4) (layer "B.Cu") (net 6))
 (segment (start 146.6075 121.788) (end 147.9175 123.098) (width 0.4) (layer "B.Cu") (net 9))
 (segment (start 146.6075 105.975) (end 146.6075 121.788) (width 0.4) (layer "B.Cu") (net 9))
 (segment (start 141.5985 124.374) (end 140.3225 123.098) (width 0.4) (layer "B.Cu") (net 9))
 (segment (start 147.9175 123.098) (end 146.6415 124.374) (width 0.4) (layer "B.Cu") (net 9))
 (segment (start 146.6415 124.374) (end 141.5985 124.374) (width 0.4) (layer "B.Cu") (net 9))
 (segment (start 147.7625 87.28) (end 147.7625 87.86) (width 0.4) (layer "B.Cu") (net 10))
 (segment (start 148.71 99.52) (end 148.71 105.1425) (width 0.4) (layer "B.Cu") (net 10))
 (segment (start 147.7625 87.86) (end 149.7025 89.8) (width 0.4) (layer "B.Cu") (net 10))
 (segment (start 148.02 93.5) (end 148.02 98.83) (width 0.4) (layer "B.Cu") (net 10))
 (segment (start 149.7025 91.8175) (end 148.02 93.5) (width 0.4) (layer "B.Cu") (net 10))
 (segment (start 148.02 98.83) (end 148.71 99.52) (width 0.4) (layer "B.Cu") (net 10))
 (segment (start 149.7025 89.22) (end 149.7025 89.8) (width 0.25) (layer "B.Cu") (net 10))
 (segment (start 149.7025 89.8) (end 149.7025 91.8175) (width 0.4) (layer "B.Cu") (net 10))
 (segment (start 148.71 105.1425) (end 147.8775 105.975) (width 0.4) (layer "B.Cu") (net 10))
 (segment (start 140.2575 101.025) (end 140.2575 105.975) (width 0.2) (layer "B.Cu") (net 8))
 (segment (start 140.2575 100.1275) (end 140.2575 101.025) (width 0.2) (layer "B.Cu") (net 8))
 (segment (start 139.02 98.89) (end 140.2575 100.1275) (width 0.2) (layer "B.Cu") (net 8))
 (segment (start 144.9 98.71) (end 144.9 100.5875) (width 0.2) (layer "B.Cu") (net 11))
 (segment (start 145.3375 100.6225) (end 145.3375 101.025) (width 0.2) (layer "B.Cu") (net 11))
 (segment (start 144.9 96.71) (end 144.88 96.69) (width 0.2) (layer "B.Cu") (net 11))
 (segment (start 144.9 100.5875) (end 145.3375 101.025) (width 0.2) (layer "B.Cu") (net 11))
 (segment (start 144.9 98.71) (end 144.9 96.71) (width 0.2) (layer "B.Cu") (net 11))
 (segment (start 137.994 97.916) (end 137.994 100.966) (width 0.2) (layer "B.Cu") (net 12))
 (segment (start 139.73016 97.791) (end 140.85 96.67116) (width 0.2) (layer "B.Cu") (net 12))
 (segment (start 136.92 103.61) (end 136.92 102.04) (width 0.2) (layer "B.Cu") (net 12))
 (segment (start 140.85 96.67116) (end 140.85 96.61) (width 0.2) (layer "B.Cu") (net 12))
 (segment (start 140.85 96.61) (end 140.85 97.02813) (width 0.3) (layer "B.Cu") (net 12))
 (segment (start 138.119 97.791) (end 137.994 97.916) (width 0.2) (layer "B.Cu") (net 12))
 (segment (start 138.119 97.791) (end 139.73016 97.791) (width 0.2) (layer "B.Cu") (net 12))
 (segment (start 137.994 100.966) (end 136.92 102.04) (width 0.2) (layer "B.Cu") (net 12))
 (segment (start 142.7975 103.4675) (end 142.745 103.52) (width 0.2) (layer "F.Cu") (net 2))
 (via (at 142.745 103.52) (size 0.6) (drill 0.3) (layers "F.Cu" "B.Cu") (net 2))
 (segment (start 142.7975 101.1175) (end 142.745 101.17) (width 0.2) (layer "B.Cu") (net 2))
 (segment (start 142.745 101.17) (end 142.745 103.52) (width 0.2) (layer "B.Cu") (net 2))
 (segment (start 142.72 100.9475) (end 142.7975 101.025) (width 0.2) (layer "B.Cu") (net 2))
 (segment (start 142.7975 101.025) (end 142.7975 101.1175) (width 0.2) (layer "B.Cu") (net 2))
 (segment (start 142.75 96.61) (end 142.75 98.61) (width 0.2) (layer "B.Cu") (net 2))
 (segment (start 142.75 98.61) (end 142.72 98.64) (width 0.2) (layer "B.Cu") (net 2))
 (segment (start 142.72 98.64) (end 142.72 100.9475) (width 0.2) (layer "B.Cu") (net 2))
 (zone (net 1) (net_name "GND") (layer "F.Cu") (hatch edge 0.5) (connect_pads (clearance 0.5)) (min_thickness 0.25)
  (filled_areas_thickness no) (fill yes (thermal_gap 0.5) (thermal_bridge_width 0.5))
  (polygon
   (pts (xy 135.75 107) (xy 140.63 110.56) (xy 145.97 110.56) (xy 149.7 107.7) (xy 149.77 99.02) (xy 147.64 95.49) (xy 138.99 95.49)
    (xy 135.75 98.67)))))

